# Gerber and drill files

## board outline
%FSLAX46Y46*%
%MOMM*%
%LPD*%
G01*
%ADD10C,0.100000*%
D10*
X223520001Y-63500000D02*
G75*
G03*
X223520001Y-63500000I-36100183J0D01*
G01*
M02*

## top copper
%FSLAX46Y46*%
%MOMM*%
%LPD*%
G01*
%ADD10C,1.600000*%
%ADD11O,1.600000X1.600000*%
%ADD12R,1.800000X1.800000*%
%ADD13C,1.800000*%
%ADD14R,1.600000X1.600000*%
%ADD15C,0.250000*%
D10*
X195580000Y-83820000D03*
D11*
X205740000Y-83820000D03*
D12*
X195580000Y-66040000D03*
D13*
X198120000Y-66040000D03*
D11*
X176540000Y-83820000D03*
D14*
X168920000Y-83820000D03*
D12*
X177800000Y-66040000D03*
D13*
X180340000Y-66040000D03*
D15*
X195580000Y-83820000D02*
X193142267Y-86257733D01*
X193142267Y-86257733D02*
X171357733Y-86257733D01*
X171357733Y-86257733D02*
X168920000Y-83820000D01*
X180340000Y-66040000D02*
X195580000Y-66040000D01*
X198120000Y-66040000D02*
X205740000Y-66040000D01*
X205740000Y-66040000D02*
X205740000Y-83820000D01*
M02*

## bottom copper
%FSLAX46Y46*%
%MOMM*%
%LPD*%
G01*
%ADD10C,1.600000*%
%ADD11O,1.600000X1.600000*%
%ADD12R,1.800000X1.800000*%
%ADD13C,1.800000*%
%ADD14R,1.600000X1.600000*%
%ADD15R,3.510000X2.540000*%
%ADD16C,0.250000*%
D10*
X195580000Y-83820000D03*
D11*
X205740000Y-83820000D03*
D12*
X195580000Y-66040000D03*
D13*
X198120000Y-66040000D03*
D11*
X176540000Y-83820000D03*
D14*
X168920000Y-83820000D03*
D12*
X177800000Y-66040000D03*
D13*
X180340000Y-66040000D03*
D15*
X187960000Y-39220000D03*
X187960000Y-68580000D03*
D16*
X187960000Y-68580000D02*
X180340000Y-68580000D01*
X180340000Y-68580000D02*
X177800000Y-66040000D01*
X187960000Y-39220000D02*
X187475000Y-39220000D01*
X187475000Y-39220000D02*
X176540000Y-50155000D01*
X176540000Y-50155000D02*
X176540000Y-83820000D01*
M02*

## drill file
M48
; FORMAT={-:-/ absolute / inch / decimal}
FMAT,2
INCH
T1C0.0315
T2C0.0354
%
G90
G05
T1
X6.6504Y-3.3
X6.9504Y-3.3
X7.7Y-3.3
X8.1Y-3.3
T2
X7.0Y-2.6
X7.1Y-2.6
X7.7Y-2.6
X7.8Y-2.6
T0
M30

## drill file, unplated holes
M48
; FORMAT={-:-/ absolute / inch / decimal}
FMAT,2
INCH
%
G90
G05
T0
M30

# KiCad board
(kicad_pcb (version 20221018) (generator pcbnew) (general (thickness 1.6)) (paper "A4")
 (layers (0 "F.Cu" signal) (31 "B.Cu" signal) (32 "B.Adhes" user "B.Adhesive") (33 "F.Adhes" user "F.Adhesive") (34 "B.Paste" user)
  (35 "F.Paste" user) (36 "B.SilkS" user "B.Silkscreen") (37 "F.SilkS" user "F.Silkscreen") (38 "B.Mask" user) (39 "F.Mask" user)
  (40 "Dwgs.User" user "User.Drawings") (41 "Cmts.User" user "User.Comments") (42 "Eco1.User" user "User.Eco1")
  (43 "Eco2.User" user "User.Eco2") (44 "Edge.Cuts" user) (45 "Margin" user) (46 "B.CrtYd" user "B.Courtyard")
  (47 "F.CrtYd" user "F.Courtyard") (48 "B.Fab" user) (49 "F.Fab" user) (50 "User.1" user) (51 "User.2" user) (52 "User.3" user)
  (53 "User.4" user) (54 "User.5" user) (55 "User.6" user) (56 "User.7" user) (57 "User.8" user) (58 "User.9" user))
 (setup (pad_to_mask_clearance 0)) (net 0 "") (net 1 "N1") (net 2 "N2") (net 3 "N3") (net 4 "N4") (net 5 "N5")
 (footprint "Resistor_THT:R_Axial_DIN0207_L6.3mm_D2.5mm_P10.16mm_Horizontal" (layer "F.Cu") (at 195.58 83.82)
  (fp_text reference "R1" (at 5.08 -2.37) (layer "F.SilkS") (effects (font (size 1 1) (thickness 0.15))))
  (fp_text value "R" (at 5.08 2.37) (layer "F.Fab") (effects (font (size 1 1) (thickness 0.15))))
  (pad "1" thru_hole circle (at 0 0) (size 1.6 1.6) (drill 0.8) (layers "*.Cu" "*.Mask") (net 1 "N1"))
  (pad "2" thru_hole oval (at 10.16 0) (size 1.6 1.6) (drill 0.8) (layers "*.Cu" "*.Mask") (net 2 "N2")))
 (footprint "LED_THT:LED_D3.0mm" (layer "F.Cu") (at 195.58 66.04)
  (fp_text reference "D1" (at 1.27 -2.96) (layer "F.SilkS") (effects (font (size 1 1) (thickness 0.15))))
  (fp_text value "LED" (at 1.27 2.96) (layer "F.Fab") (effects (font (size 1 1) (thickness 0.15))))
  (pad "1" thru_hole rect (at 0 0) (size 1.8 1.8) (drill 0.9) (layers "*.Cu" "*.Mask") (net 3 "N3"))
  (pad "2" thru_hole circle (at 2.54 0) (size 1.8 1.8) (drill 0.9) (layers "*.Cu" "*.Mask") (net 2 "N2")))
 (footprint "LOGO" (layer "F.Cu") (at 187.96 63.5)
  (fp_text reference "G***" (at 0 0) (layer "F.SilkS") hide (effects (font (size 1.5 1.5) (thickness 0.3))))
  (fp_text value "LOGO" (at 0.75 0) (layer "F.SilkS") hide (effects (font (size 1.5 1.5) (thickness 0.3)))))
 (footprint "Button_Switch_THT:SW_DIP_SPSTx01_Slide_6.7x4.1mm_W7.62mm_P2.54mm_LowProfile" (layer "F.Cu") (at 168.92 83.82)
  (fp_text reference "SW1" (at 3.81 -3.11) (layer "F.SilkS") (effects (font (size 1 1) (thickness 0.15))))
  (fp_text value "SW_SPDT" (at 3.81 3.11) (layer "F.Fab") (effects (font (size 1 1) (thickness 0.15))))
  (pad "1" thru_hole rect (at 0 0) (size 1.6 1.6) (drill 0.8) (layers "*.Cu" "*.Mask") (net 1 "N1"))
  (pad "2" thru_hole oval (at 7.62 0) (size 1.6 1.6) (drill 0.8) (layers "*.Cu" "*.Mask") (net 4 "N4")))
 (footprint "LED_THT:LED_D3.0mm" (layer "F.Cu") (at 177.8 66.04)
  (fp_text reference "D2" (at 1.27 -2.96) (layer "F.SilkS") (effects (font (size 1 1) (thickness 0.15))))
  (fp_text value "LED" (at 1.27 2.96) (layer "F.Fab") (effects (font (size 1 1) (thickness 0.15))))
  (pad "1" thru_hole rect (at 0 0) (size 1.8 1.8) (drill 0.9) (layers "*.Cu" "*.Mask") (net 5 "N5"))
  (pad "2" thru_hole circle (at 2.54 0) (size 1.8 1.8) (drill 0.9) (layers "*.Cu" "*.Mask") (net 3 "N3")))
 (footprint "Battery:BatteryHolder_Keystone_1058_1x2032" (layer "B.Cu") (at 187.96 53.9 -90)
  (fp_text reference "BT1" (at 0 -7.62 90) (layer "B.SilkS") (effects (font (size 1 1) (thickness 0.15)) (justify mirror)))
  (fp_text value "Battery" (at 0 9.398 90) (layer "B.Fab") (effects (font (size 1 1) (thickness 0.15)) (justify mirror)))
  (pad "1" smd rect (at -14.68 0 270) (size 2.54 3.51) (layers "B.Cu" "B.Paste" "B.Mask") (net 4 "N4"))
  (pad "2" smd rect (at 14.68 0 270) (size 2.54 3.51) (layers "B.Cu" "B.Paste" "B.Mask") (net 5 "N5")))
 (gr_circle (center 187.419818 63.5) (end 215.359818 86.36) (stroke (width 0.1) (type default)) (fill none) (layer "Edge.Cuts"))
 (segment (start 193.142267 86.257733) (end 171.357733 86.257733) (width 0.25) (layer "F.Cu") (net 1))
 (segment (start 171.357733 86.257733) (end 168.92 83.82) (width 0.25) (layer "F.Cu") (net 1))
 (segment (start 195.58 83.82) (end 193.142267 86.257733) (width 0.25) (layer "F.Cu") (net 1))
 (segment (start 205.74 66.04) (end 205.74 83.82) (width 0.25) (layer "F.Cu") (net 2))
 (segment (start 198.12 66.04) (end 205.74 66.04) (width 0.25) (layer "F.Cu") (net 2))
 (segment (start 180.34 66.04) (end 195.58 66.04) (width 0.25) (layer "F.Cu") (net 3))
 (segment (start 187.96 68.58) (end 180.34 68.58) (width 0.25) (layer "B.Cu") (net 5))
 (segment (start 180.34 68.58) (end 177.8 66.04) (width 0.25) (layer "B.Cu") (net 5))
 (segment (start 187.475 39.22) (end 176.54 50.155) (width 0.25) (layer "B.Cu") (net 4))
 (segment (start 176.54 50.155) (end 176.54 83.82) (width 0.25) (layer "B.Cu") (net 4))
 (segment (start 187.96 39.22) (end 187.475 39.22) (width 0.25) (layer "B.Cu") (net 4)))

